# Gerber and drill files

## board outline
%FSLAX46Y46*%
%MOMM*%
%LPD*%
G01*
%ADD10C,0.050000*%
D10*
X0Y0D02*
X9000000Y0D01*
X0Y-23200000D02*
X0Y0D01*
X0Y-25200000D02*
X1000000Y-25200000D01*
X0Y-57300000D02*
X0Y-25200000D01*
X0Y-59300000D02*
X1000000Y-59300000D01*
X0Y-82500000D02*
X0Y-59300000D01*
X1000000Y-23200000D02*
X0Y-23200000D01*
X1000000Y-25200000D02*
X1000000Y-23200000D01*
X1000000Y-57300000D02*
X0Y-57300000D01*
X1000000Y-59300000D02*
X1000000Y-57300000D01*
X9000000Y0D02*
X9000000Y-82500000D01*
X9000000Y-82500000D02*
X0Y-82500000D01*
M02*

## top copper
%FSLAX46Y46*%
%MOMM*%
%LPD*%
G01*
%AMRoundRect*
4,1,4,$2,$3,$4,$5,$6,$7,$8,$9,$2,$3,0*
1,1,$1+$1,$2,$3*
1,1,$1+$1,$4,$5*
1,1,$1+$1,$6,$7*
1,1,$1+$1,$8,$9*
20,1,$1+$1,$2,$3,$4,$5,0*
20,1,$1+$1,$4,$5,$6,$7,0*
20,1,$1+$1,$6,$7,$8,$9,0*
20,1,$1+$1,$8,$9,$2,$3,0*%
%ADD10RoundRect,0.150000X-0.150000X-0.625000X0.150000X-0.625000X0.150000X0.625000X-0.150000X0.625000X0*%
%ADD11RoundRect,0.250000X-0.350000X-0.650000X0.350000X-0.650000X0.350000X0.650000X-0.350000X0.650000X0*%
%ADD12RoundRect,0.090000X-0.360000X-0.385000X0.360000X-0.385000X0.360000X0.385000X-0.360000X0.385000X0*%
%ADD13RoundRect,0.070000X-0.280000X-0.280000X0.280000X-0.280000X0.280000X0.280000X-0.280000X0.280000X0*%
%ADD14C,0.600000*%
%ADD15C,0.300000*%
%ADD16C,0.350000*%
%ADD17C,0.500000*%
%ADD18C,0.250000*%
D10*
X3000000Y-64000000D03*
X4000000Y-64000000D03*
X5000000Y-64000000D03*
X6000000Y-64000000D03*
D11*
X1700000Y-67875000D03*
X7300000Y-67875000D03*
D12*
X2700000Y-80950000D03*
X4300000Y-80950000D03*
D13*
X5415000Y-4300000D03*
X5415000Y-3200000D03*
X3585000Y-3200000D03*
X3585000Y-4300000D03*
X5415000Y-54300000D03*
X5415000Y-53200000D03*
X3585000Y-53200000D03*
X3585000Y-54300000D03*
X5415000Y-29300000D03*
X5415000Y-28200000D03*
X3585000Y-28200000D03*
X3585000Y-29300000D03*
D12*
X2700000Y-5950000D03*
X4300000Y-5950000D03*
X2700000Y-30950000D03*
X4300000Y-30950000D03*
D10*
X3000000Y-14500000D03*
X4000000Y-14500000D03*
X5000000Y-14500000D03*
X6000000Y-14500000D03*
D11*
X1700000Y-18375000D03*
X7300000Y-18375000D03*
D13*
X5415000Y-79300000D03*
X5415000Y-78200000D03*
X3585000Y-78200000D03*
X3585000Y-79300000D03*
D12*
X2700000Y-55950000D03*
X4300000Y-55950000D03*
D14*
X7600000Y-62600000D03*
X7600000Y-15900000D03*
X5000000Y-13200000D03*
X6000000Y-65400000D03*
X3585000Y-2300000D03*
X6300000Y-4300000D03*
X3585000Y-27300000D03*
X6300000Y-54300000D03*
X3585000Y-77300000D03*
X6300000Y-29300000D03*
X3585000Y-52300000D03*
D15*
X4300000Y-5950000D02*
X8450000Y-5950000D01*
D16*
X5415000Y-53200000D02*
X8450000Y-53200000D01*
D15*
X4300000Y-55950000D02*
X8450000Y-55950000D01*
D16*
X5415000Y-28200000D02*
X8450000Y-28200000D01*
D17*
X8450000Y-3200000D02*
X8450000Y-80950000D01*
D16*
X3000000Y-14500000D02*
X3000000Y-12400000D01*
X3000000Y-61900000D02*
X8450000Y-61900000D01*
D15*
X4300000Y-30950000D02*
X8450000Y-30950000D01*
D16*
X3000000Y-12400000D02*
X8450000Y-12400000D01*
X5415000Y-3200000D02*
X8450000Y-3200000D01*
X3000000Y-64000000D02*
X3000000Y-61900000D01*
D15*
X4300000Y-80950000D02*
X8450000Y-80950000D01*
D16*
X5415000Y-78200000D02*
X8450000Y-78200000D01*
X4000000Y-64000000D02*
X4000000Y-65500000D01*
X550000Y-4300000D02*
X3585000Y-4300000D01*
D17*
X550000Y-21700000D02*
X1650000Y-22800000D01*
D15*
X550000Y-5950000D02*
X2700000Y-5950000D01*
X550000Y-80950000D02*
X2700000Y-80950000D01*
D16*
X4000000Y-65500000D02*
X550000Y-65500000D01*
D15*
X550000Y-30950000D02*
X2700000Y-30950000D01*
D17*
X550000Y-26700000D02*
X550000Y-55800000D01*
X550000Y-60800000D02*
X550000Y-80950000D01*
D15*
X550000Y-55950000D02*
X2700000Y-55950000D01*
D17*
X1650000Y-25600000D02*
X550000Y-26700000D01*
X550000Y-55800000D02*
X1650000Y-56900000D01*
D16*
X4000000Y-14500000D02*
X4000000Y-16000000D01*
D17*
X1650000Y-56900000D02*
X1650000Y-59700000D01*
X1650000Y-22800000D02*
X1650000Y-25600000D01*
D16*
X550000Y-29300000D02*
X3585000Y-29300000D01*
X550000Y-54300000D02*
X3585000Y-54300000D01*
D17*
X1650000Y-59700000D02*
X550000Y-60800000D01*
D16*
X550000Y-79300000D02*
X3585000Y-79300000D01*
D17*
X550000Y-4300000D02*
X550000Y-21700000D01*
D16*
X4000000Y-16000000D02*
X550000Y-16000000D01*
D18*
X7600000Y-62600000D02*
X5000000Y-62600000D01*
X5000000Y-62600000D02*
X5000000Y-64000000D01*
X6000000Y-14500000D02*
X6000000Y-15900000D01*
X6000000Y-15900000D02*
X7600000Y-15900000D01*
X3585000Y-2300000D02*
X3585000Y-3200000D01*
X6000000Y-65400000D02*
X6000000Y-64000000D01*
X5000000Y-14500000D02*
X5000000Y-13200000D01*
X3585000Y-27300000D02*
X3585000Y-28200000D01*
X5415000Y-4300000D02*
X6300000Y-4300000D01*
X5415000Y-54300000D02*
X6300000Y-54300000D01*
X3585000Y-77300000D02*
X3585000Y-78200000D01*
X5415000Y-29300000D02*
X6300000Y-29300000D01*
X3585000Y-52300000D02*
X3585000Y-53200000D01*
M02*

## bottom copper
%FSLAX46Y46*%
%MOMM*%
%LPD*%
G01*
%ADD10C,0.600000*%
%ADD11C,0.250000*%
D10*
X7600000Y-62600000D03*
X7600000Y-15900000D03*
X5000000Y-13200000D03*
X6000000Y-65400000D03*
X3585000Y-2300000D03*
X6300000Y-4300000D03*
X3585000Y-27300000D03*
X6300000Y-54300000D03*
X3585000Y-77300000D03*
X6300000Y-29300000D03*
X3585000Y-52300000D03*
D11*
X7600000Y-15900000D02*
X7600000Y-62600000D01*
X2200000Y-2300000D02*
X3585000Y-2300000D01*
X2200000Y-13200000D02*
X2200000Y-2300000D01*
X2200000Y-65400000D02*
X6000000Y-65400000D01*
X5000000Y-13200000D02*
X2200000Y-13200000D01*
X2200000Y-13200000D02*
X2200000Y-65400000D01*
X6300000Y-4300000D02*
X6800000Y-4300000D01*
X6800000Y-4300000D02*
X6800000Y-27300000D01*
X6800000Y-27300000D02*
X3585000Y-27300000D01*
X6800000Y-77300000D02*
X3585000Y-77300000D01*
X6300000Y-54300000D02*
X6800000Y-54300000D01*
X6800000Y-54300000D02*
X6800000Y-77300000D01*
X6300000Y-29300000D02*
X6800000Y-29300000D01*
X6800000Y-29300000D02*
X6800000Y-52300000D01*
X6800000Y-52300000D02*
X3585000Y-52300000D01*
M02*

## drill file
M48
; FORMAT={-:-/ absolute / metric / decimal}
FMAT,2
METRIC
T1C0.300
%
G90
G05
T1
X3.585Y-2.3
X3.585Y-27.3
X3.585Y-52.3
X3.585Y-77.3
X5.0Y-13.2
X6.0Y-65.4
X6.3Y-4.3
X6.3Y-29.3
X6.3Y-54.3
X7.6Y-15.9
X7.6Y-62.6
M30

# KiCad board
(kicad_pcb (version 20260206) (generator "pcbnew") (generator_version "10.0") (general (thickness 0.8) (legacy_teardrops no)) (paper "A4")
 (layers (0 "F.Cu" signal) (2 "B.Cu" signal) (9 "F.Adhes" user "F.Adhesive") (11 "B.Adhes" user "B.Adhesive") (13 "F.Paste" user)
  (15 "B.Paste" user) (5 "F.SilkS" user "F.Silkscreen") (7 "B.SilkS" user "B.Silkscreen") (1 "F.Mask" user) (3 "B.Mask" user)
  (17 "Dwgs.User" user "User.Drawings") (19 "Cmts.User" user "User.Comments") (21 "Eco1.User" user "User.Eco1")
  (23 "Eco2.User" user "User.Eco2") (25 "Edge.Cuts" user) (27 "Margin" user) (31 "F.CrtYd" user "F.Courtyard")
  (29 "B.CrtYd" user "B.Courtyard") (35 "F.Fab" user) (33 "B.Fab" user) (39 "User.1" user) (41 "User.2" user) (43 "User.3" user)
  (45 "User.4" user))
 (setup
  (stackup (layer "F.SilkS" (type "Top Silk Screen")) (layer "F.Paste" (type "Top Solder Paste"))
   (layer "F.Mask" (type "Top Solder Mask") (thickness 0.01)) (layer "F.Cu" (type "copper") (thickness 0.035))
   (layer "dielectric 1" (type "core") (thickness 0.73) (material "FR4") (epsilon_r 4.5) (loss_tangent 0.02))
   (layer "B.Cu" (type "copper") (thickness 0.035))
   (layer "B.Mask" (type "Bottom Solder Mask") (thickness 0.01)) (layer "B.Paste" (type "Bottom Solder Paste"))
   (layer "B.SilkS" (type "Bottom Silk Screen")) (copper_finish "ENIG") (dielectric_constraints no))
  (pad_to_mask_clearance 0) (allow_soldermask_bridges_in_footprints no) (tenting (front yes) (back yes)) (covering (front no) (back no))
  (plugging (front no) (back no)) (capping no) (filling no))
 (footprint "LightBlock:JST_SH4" (layer "F.Cu") (at 4.5 66)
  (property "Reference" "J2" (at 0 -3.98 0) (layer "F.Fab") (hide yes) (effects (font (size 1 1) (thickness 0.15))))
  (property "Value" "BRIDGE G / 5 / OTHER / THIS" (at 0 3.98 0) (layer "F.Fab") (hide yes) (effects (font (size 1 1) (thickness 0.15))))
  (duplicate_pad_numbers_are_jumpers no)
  (pad "1" smd roundrect (at -1.5 -2) (size 0.6 1.55) (layers "F.Cu" "F.Mask" "F.Paste") (roundrect_rratio 0.25) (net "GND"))
  (pad "2" smd roundrect (at -0.5 -2) (size 0.6 1.55) (layers "F.Cu" "F.Mask" "F.Paste") (roundrect_rratio 0.25) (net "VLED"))
  (pad "3" smd roundrect (at 0.5 -2) (size 0.6 1.55) (layers "F.Cu" "F.Mask" "F.Paste") (roundrect_rratio 0.25) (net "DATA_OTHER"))
  (pad "4" smd roundrect (at 1.5 -2) (size 0.6 1.55) (layers "F.Cu" "F.Mask" "F.Paste") (roundrect_rratio 0.25) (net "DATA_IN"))
  (pad "MP" smd roundrect (at -2.8 1.875) (size 1.2 1.8) (layers "F.Cu" "F.Mask" "F.Paste") (roundrect_rratio 0.208333))
  (pad "MP" smd roundrect (at 2.8 1.875) (size 1.2 1.8) (layers "F.Cu" "F.Mask" "F.Paste") (roundrect_rratio 0.208333)))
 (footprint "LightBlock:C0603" (layer "F.Cu") (at 3.5 80.95)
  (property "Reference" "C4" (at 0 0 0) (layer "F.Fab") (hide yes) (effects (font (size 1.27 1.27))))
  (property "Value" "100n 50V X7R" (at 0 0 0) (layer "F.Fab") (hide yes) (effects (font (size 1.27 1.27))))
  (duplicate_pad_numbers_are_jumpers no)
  (pad "1" smd roundrect (at -0.8 0) (size 0.9 0.95) (layers "F.Cu" "F.Mask" "F.Paste") (roundrect_rratio 0.1) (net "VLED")
   (thermal_bridge_angle 45))
  (pad "2" smd roundrect (at 0.8 0) (size 0.9 0.95) (layers "F.Cu" "F.Mask" "F.Paste") (roundrect_rratio 0.1) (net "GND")
   (thermal_bridge_angle 45)))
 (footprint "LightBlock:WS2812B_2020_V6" (layer "F.Cu") (at 4.5 3.75)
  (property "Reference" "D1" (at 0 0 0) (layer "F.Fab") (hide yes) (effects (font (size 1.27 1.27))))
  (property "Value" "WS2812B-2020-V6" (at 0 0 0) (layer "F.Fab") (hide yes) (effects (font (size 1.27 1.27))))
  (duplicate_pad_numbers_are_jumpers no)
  (pad "1" smd roundrect (at 0.915 0.55) (size 0.7 0.7) (layers "F.Cu" "F.Mask" "F.Paste") (roundrect_rratio 0.1) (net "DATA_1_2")
   (thermal_bridge_angle 45))
  (pad "2" smd roundrect (at 0.915 -0.55) (size 0.7 0.7) (layers "F.Cu" "F.Mask" "F.Paste") (roundrect_rratio 0.1) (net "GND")
   (thermal_bridge_angle 45))
  (pad "3" smd roundrect (at -0.915 -0.55) (size 0.7 0.7) (layers "F.Cu" "F.Mask" "F.Paste") (roundrect_rratio 0.1) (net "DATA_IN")
   (thermal_bridge_angle 45))
  (pad "4" smd roundrect (at -0.915 0.55) (size 0.7 0.7) (layers "F.Cu" "F.Mask" "F.Paste") (roundrect_rratio 0.1) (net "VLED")
   (thermal_bridge_angle 45)))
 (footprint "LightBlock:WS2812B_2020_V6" (layer "F.Cu") (at 4.5 53.75)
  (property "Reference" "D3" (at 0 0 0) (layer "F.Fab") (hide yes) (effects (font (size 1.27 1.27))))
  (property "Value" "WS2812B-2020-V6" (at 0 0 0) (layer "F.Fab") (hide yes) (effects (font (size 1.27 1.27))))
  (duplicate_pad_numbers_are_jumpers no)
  (pad "1" smd roundrect (at 0.915 0.55) (size 0.7 0.7) (layers "F.Cu" "F.Mask" "F.Paste") (roundrect_rratio 0.1) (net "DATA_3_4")
   (thermal_bridge_angle 45))
  (pad "2" smd roundrect (at 0.915 -0.55) (size 0.7 0.7) (layers "F.Cu" "F.Mask" "F.Paste") (roundrect_rratio 0.1) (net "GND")
   (thermal_bridge_angle 45))
  (pad "3" smd roundrect (at -0.915 -0.55) (size 0.7 0.7) (layers "F.Cu" "F.Mask" "F.Paste") (roundrect_rratio 0.1) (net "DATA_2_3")
   (thermal_bridge_angle 45))
  (pad "4" smd roundrect (at -0.915 0.55) (size 0.7 0.7) (layers "F.Cu" "F.Mask" "F.Paste") (roundrect_rratio 0.1) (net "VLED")
   (thermal_bridge_angle 45)))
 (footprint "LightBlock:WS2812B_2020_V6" (layer "F.Cu") (at 4.5 28.75)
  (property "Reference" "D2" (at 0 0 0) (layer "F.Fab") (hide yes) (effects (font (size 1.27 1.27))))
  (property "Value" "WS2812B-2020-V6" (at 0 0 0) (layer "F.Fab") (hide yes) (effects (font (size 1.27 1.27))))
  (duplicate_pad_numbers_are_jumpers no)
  (pad "1" smd roundrect (at 0.915 0.55) (size 0.7 0.7) (layers "F.Cu" "F.Mask" "F.Paste") (roundrect_rratio 0.1) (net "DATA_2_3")
   (thermal_bridge_angle 45))
  (pad "2" smd roundrect (at 0.915 -0.55) (size 0.7 0.7) (layers "F.Cu" "F.Mask" "F.Paste") (roundrect_rratio 0.1) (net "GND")
   (thermal_bridge_angle 45))
  (pad "3" smd roundrect (at -0.915 -0.55) (size 0.7 0.7) (layers "F.Cu" "F.Mask" "F.Paste") (roundrect_rratio 0.1) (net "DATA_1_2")
   (thermal_bridge_angle 45))
  (pad "4" smd roundrect (at -0.915 0.55) (size 0.7 0.7) (layers "F.Cu" "F.Mask" "F.Paste") (roundrect_rratio 0.1) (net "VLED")
   (thermal_bridge_angle 45)))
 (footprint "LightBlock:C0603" (layer "F.Cu") (at 3.5 5.95)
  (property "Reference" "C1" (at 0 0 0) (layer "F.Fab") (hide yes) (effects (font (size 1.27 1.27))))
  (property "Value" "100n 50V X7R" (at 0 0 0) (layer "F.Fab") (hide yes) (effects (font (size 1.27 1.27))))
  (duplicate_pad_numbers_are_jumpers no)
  (pad "1" smd roundrect (at -0.8 0) (size 0.9 0.95) (layers "F.Cu" "F.Mask" "F.Paste") (roundrect_rratio 0.1) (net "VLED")
   (thermal_bridge_angle 45))
  (pad "2" smd roundrect (at 0.8 0) (size 0.9 0.95) (layers "F.Cu" "F.Mask" "F.Paste") (roundrect_rratio 0.1) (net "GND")
   (thermal_bridge_angle 45)))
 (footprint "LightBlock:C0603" (layer "F.Cu") (at 3.5 30.95)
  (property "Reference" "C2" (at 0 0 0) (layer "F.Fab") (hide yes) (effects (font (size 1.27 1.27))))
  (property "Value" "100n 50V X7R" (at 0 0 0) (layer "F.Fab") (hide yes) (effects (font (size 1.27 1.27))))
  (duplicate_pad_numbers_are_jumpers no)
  (pad "1" smd roundrect (at -0.8 0) (size 0.9 0.95) (layers "F.Cu" "F.Mask" "F.Paste") (roundrect_rratio 0.1) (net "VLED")
   (thermal_bridge_angle 45))
  (pad "2" smd roundrect (at 0.8 0) (size 0.9 0.95) (layers "F.Cu" "F.Mask" "F.Paste") (roundrect_rratio 0.1) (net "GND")
   (thermal_bridge_angle 45)))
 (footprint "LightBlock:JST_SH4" (layer "F.Cu") (at 4.5 16.5)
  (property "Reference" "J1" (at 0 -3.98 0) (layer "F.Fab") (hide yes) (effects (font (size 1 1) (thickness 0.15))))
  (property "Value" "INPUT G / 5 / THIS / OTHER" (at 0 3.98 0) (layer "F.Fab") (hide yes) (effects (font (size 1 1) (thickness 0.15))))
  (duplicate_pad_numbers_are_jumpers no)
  (pad "1" smd roundrect (at -1.5 -2) (size 0.6 1.55) (layers "F.Cu" "F.Mask" "F.Paste") (roundrect_rratio 0.25) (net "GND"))
  (pad "2" smd roundrect (at -0.5 -2) (size 0.6 1.55) (layers "F.Cu" "F.Mask" "F.Paste") (roundrect_rratio 0.25) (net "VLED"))
  (pad "3" smd roundrect (at 0.5 -2) (size 0.6 1.55) (layers "F.Cu" "F.Mask" "F.Paste") (roundrect_rratio 0.25) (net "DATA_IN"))
  (pad "4" smd roundrect (at 1.5 -2) (size 0.6 1.55) (layers "F.Cu" "F.Mask" "F.Paste") (roundrect_rratio 0.25) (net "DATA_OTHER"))
  (pad "MP" smd roundrect (at -2.8 1.875) (size 1.2 1.8) (layers "F.Cu" "F.Mask" "F.Paste") (roundrect_rratio 0.208333))
  (pad "MP" smd roundrect (at 2.8 1.875) (size 1.2 1.8) (layers "F.Cu" "F.Mask" "F.Paste") (roundrect_rratio 0.208333)))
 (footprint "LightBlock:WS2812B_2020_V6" (layer "F.Cu") (at 4.5 78.75)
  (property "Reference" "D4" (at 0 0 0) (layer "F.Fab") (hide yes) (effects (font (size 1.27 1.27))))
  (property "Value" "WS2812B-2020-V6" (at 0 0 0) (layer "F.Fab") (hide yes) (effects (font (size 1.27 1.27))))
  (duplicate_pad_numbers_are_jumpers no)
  (pad "1" smd roundrect (at 0.915 0.55) (size 0.7 0.7) (layers "F.Cu" "F.Mask" "F.Paste") (roundrect_rratio 0.1) (thermal_bridge_angle 45))
  (pad "2" smd roundrect (at 0.915 -0.55) (size 0.7 0.7) (layers "F.Cu" "F.Mask" "F.Paste") (roundrect_rratio 0.1) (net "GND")
   (thermal_bridge_angle 45))
  (pad "3" smd roundrect (at -0.915 -0.55) (size 0.7 0.7) (layers "F.Cu" "F.Mask" "F.Paste") (roundrect_rratio 0.1) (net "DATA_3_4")
   (thermal_bridge_angle 45))
  (pad "4" smd roundrect (at -0.915 0.55) (size 0.7 0.7) (layers "F.Cu" "F.Mask" "F.Paste") (roundrect_rratio 0.1) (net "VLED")
   (thermal_bridge_angle 45)))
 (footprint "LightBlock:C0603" (layer "F.Cu") (at 3.5 55.95)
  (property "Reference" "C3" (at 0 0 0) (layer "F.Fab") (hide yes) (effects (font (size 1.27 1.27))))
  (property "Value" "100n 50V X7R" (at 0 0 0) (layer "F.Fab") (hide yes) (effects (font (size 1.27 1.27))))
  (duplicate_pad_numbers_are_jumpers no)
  (pad "1" smd roundrect (at -0.8 0) (size 0.9 0.95) (layers "F.Cu" "F.Mask" "F.Paste") (roundrect_rratio 0.1) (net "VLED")
   (thermal_bridge_angle 45))
  (pad "2" smd roundrect (at 0.8 0) (size 0.9 0.95) (layers "F.Cu" "F.Mask" "F.Paste") (roundrect_rratio 0.1) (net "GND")
   (thermal_bridge_angle 45)))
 (gr_line (start 0 0) (end 9 0) (stroke (width 0.05) (type default)) (layer "Edge.Cuts"))
 (gr_line (start 0 23.2) (end 0 0) (stroke (width 0.05) (type default)) (layer "Edge.Cuts"))
 (gr_line (start 0 25.2) (end 1 25.2) (stroke (width 0.05) (type default)) (layer "Edge.Cuts"))
 (gr_line (start 0 57.3) (end 0 25.2) (stroke (width 0.05) (type default)) (layer "Edge.Cuts"))
 (gr_line (start 0 59.3) (end 1 59.3) (stroke (width 0.05) (type default)) (layer "Edge.Cuts"))
 (gr_line (start 0 82.5) (end 0 59.3) (stroke (width 0.05) (type default)) (layer "Edge.Cuts"))
 (gr_line (start 1 23.2) (end 0 23.2) (stroke (width 0.05) (type default)) (layer "Edge.Cuts"))
 (gr_line (start 1 25.2) (end 1 23.2) (stroke (width 0.05) (type default)) (layer "Edge.Cuts"))
 (gr_line (start 1 57.3) (end 0 57.3) (stroke (width 0.05) (type default)) (layer "Edge.Cuts"))
 (gr_line (start 1 59.3) (end 1 57.3) (stroke (width 0.05) (type default)) (layer "Edge.Cuts"))
 (gr_line (start 9 0) (end 9 82.5) (stroke (width 0.05) (type default)) (layer "Edge.Cuts"))
 (gr_line (start 9 82.5) (end 0 82.5) (stroke (width 0.05) (type default)) (layer "Edge.Cuts"))
 (segment (start 4.3 5.95) (end 8.45 5.95) (width 0.3) (layer "F.Cu") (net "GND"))
 (segment (start 5.415 53.2) (end 8.45 53.2) (width 0.35) (layer "F.Cu") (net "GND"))
 (segment (start 4.3 55.95) (end 8.45 55.95) (width 0.3) (layer "F.Cu") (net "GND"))
 (segment (start 5.415 28.2) (end 8.45 28.2) (width 0.35) (layer "F.Cu") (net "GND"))
 (segment (start 8.45 3.2) (end 8.45 80.95) (width 0.5) (layer "F.Cu") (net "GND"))
 (segment (start 3 14.5) (end 3 12.4) (width 0.35) (layer "F.Cu") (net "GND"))
 (segment (start 3 61.9) (end 8.45 61.9) (width 0.35) (layer "F.Cu") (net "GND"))
 (segment (start 4.3 30.95) (end 8.45 30.95) (width 0.3) (layer "F.Cu") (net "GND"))
 (segment (start 3 12.4) (end 8.45 12.4) (width 0.35) (layer "F.Cu") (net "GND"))
 (segment (start 5.415 3.2) (end 8.45 3.2) (width 0.35) (layer "F.Cu") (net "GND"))
 (segment (start 3 64) (end 3 61.9) (width 0.35) (layer "F.Cu") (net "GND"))
 (segment (start 4.3 80.95) (end 8.45 80.95) (width 0.3) (layer "F.Cu") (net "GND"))
 (segment (start 5.415 78.2) (end 8.45 78.2) (width 0.35) (layer "F.Cu") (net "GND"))
 (segment (start 4 64) (end 4 65.5) (width 0.35) (layer "F.Cu") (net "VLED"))
 (segment (start 0.55 4.3) (end 3.585 4.3) (width 0.35) (layer "F.Cu") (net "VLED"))
 (segment (start 0.55 21.7) (end 1.65 22.8) (width 0.5) (layer "F.Cu") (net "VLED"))
 (segment (start 0.55 5.95) (end 2.7 5.95) (width 0.3) (layer "F.Cu") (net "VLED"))
 (segment (start 0.55 80.95) (end 2.7 80.95) (width 0.3) (layer "F.Cu") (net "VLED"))
 (segment (start 4 65.5) (end 0.55 65.5) (width 0.35) (layer "F.Cu") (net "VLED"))
 (segment (start 0.55 30.95) (end 2.7 30.95) (width 0.3) (layer "F.Cu") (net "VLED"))
 (segment (start 0.55 26.7) (end 0.55 55.8) (width 0.5) (layer "F.Cu") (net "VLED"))
 (segment (start 0.55 60.8) (end 0.55 80.95) (width 0.5) (layer "F.Cu") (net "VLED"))
 (segment (start 0.55 55.95) (end 2.7 55.95) (width 0.3) (layer "F.Cu") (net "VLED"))
 (segment (start 1.65 25.6) (end 0.55 26.7) (width 0.5) (layer "F.Cu") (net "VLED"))
 (segment (start 0.55 55.8) (end 1.65 56.9) (width 0.5) (layer "F.Cu") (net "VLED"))
 (segment (start 4 14.5) (end 4 16) (width 0.35) (layer "F.Cu") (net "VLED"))
 (segment (start 1.65 56.9) (end 1.65 59.7) (width 0.5) (layer "F.Cu") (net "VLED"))
 (segment (start 1.65 22.8) (end 1.65 25.6) (width 0.5) (layer "F.Cu") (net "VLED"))
 (segment (start 0.55 29.3) (end 3.585 29.3) (width 0.35) (layer "F.Cu") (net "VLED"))
 (segment (start 0.55 54.3) (end 3.585 54.3) (width 0.35) (layer "F.Cu") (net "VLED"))
 (segment (start 1.65 59.7) (end 0.55 60.8) (width 0.5) (layer "F.Cu") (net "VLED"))
 (segment (start 0.55 79.3) (end 3.585 79.3) (width 0.35) (layer "F.Cu") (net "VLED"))
 (segment (start 0.55 4.3) (end 0.55 21.7) (width 0.5) (layer "F.Cu") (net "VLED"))
 (segment (start 4 16) (end 0.55 16) (width 0.35) (layer "F.Cu") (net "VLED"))
 (segment (start 7.6 62.6) (end 5 62.6) (width 0.25) (layer "F.Cu") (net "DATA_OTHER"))
 (segment (start 5 62.6) (end 5 64) (width 0.25) (layer "F.Cu") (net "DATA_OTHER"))
 (segment (start 6 14.5) (end 6 15.9) (width 0.25) (layer "F.Cu") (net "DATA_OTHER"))
 (segment (start 6 15.9) (end 7.6 15.9) (width 0.25) (layer "F.Cu") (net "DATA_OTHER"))
 (via (at 7.6 62.6) (size 0.6) (drill 0.3) (layers "F.Cu" "B.Cu") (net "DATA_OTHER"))
 (via (at 7.6 15.9) (size 0.6) (drill 0.3) (layers "F.Cu" "B.Cu") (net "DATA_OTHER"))
 (segment (start 7.6 15.9) (end 7.6 62.6) (width 0.25) (layer "B.Cu") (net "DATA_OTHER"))
 (segment (start 3.585 2.3) (end 3.585 3.2) (width 0.25) (layer "F.Cu") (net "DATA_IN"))
 (segment (start 6 65.4) (end 6 64) (width 0.25) (layer "F.Cu") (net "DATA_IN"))
 (segment (start 5 14.5) (end 5 13.2) (width 0.25) (layer "F.Cu") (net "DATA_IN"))
 (via (at 5 13.2) (size 0.6) (drill 0.3) (layers "F.Cu" "B.Cu") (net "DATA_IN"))
 (via (at 6 65.4) (size 0.6) (drill 0.3) (layers "F.Cu" "B.Cu") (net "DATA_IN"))
 (via (at 3.585 2.3) (size 0.6) (drill 0.3) (layers "F.Cu" "B.Cu") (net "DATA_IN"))
 (segment (start 2.2 2.3) (end 3.585 2.3) (width 0.25) (layer "B.Cu") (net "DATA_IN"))
 (segment (start 2.2 13.2) (end 2.2 2.3) (width 0.25) (layer "B.Cu") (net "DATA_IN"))
 (segment (start 2.2 65.4) (end 6 65.4) (width 0.25) (layer "B.Cu") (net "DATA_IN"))
 (segment (start 5 13.2) (end 2.2 13.2) (width 0.25) (layer "B.Cu") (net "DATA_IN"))
 (segment (start 2.2 13.2) (end 2.2 65.4) (width 0.25) (layer "B.Cu") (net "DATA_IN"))
 (segment (start 3.585 27.3) (end 3.585 28.2) (width 0.25) (layer "F.Cu") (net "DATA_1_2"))
 (segment (start 5.415 4.3) (end 6.3 4.3) (width 0.25) (layer "F.Cu") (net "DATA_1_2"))
 (via (at 6.3 4.3) (size 0.6) (drill 0.3) (layers "F.Cu" "B.Cu") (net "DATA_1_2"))
 (via (at 3.585 27.3) (size 0.6) (drill 0.3) (layers "F.Cu" "B.Cu") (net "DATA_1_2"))
 (segment (start 6.3 4.3) (end 6.8 4.3) (width 0.25) (layer "B.Cu") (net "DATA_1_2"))
 (segment (start 6.8 4.3) (end 6.8 27.3) (width 0.25) (layer "B.Cu") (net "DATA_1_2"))
 (segment (start 6.8 27.3) (end 3.585 27.3) (width 0.25) (layer "B.Cu") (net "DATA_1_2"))
 (segment (start 5.415 54.3) (end 6.3 54.3) (width 0.25) (layer "F.Cu") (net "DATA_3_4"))
 (segment (start 3.585 77.3) (end 3.585 78.2) (width 0.25) (layer "F.Cu") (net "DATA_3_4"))
 (via (at 6.3 54.3) (size 0.6) (drill 0.3) (layers "F.Cu" "B.Cu") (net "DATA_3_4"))
 (via (at 3.585 77.3) (size 0.6) (drill 0.3) (layers "F.Cu" "B.Cu") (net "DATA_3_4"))
 (segment (start 6.8 77.3) (end 3.585 77.3) (width 0.25) (layer "B.Cu") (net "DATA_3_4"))
 (segment (start 6.3 54.3) (end 6.8 54.3) (width 0.25) (layer "B.Cu") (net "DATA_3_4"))
 (segment (start 6.8 54.3) (end 6.8 77.3) (width 0.25) (layer "B.Cu") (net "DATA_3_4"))
 (segment (start 5.415 29.3) (end 6.3 29.3) (width 0.25) (layer "F.Cu") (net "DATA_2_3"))
 (segment (start 3.585 52.3) (end 3.585 53.2) (width 0.25) (layer "F.Cu") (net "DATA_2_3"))
 (via (at 6.3 29.3) (size 0.6) (drill 0.3) (layers "F.Cu" "B.Cu") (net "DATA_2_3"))
 (via (at 3.585 52.3) (size 0.6) (drill 0.3) (layers "F.Cu" "B.Cu") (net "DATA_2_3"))
 (segment (start 6.3 29.3) (end 6.8 29.3) (width 0.25) (layer "B.Cu") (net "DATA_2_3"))
 (segment (start 6.8 29.3) (end 6.8 52.3) (width 0.25) (layer "B.Cu") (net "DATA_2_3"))
 (segment (start 6.8 52.3) (end 3.585 52.3) (width 0.25) (layer "B.Cu") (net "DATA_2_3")))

